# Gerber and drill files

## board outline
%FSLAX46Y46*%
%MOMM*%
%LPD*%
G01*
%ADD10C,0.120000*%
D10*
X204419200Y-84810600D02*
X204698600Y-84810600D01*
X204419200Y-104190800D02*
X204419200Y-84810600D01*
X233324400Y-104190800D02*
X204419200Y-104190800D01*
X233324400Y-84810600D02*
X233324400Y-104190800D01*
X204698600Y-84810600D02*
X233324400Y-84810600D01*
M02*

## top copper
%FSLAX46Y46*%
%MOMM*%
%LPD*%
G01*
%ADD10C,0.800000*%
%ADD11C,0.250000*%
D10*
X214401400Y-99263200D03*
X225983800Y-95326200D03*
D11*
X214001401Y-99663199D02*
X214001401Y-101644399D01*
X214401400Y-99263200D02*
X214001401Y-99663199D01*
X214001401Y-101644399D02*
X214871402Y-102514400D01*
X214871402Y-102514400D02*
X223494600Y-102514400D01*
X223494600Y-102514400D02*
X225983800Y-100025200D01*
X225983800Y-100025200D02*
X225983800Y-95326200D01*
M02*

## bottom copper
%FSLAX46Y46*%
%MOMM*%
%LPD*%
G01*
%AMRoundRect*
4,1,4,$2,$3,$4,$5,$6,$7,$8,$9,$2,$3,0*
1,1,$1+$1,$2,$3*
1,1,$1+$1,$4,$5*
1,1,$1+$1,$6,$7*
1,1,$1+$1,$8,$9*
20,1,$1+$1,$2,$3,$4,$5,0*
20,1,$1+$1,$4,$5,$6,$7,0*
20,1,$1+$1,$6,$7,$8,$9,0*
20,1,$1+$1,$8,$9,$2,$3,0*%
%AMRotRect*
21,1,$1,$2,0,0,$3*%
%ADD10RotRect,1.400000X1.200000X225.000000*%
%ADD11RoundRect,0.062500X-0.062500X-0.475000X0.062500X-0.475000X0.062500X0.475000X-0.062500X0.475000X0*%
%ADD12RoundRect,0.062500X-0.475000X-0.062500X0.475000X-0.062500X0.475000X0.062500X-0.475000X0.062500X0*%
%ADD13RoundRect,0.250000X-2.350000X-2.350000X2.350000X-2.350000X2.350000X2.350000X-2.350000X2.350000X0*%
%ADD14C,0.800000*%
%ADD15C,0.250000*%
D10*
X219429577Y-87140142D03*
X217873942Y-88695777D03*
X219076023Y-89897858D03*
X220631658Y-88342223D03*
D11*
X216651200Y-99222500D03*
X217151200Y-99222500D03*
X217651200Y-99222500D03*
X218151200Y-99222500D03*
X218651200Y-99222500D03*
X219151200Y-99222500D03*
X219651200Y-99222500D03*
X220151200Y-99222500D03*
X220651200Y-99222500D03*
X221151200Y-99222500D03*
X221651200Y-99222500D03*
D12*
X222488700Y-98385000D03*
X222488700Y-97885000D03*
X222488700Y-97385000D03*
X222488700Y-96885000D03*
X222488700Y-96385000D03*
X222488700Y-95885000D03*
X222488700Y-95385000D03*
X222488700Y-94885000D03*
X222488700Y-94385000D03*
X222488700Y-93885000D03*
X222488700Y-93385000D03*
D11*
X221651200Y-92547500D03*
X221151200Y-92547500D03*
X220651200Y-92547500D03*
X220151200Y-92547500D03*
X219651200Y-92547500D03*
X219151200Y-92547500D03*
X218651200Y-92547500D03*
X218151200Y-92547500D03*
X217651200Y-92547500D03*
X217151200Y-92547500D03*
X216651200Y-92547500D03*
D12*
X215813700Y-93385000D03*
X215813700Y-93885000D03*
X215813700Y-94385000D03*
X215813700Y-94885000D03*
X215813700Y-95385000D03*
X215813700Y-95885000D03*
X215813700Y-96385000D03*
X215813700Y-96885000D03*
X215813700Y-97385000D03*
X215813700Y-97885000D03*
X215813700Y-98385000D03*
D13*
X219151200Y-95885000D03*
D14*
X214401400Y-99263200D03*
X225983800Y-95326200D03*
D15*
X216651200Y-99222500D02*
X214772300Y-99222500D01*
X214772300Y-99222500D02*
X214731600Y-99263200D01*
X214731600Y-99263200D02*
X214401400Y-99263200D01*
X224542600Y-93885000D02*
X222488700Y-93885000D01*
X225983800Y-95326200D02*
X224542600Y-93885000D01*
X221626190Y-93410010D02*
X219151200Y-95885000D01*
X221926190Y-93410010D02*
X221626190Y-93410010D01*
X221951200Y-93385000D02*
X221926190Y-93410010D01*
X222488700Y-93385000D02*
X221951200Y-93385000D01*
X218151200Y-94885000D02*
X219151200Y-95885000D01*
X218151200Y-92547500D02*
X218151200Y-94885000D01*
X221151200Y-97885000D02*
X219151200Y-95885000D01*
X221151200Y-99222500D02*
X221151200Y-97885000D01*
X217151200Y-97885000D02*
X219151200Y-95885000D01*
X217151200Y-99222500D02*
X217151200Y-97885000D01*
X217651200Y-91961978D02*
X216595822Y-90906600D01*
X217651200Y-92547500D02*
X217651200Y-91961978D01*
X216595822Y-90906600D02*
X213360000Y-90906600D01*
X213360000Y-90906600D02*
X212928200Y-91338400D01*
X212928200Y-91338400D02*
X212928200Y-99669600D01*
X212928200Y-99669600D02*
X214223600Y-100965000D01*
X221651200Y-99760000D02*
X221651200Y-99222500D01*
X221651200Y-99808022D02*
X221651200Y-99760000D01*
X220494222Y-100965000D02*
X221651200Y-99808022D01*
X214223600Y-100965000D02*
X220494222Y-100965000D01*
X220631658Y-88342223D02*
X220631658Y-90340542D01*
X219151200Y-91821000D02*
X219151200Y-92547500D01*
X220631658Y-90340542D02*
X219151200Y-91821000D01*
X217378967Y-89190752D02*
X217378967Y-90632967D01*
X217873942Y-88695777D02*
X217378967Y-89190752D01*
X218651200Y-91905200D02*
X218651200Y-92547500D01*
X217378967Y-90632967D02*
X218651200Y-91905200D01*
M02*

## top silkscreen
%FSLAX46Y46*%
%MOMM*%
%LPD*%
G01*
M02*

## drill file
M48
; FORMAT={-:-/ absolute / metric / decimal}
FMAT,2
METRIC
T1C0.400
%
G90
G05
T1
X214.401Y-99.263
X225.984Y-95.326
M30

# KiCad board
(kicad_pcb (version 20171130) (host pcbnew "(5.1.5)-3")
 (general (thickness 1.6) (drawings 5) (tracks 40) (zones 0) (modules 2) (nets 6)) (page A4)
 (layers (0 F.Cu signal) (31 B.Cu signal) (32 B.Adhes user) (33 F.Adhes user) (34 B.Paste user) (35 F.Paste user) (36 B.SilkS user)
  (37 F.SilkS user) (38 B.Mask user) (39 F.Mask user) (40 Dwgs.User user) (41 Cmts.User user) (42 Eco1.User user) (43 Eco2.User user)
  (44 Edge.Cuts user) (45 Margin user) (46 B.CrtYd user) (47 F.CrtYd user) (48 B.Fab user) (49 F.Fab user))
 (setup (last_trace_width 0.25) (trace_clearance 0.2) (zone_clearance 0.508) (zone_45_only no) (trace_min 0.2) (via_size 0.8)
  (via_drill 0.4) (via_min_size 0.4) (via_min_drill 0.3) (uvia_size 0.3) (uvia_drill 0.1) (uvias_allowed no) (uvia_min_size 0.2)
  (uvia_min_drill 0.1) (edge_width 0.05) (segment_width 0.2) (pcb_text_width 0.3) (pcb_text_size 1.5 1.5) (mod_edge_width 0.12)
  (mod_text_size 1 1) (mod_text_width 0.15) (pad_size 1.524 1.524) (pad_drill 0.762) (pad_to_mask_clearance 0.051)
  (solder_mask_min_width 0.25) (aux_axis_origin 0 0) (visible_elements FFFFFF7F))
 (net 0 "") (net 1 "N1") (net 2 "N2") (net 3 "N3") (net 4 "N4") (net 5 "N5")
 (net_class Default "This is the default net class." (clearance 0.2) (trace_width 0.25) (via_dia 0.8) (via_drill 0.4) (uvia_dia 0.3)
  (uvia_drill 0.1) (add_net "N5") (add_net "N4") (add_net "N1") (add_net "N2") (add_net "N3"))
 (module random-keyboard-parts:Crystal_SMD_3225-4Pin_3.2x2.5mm (layer B.Cu) (at 219.2528 88.519 225)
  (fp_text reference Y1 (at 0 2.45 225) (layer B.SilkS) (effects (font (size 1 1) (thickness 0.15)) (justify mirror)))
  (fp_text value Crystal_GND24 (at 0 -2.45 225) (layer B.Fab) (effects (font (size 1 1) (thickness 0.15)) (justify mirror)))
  (pad 4 smd rect (at -1.1 0.85 225) (size 1.4 1.2) (layers B.Cu B.Paste B.Mask))
  (pad 3 smd rect (at 1.1 0.85 225) (size 1.4 1.2) (layers B.Cu B.Paste B.Mask) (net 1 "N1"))
  (pad 2 smd rect (at 1.1 -0.85 225) (size 1.4 1.2) (layers B.Cu B.Paste B.Mask))
  (pad 1 smd rect (at -1.1 -0.85 225) (size 1.4 1.2) (layers B.Cu B.Paste B.Mask) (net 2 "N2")))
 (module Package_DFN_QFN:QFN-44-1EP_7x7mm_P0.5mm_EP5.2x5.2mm (layer B.Cu) (at 219.1512 95.885)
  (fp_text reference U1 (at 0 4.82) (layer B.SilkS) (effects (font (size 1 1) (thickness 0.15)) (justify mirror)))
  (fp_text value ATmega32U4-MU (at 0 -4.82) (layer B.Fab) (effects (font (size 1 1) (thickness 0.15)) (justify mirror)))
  (pad 44 smd roundrect (at -2.5 3.3375) (size 0.25 1.075) (layers B.Cu B.Paste B.Mask) (roundrect_rratio 0.25) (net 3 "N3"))
  (pad 43 smd roundrect (at -2 3.3375) (size 0.25 1.075) (layers B.Cu B.Paste B.Mask) (roundrect_rratio 0.25) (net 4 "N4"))
  (pad 42 smd roundrect (at -1.5 3.3375) (size 0.25 1.075) (layers B.Cu B.Paste B.Mask) (roundrect_rratio 0.25))
  (pad 41 smd roundrect (at -1 3.3375) (size 0.25 1.075) (layers B.Cu B.Paste B.Mask) (roundrect_rratio 0.25))
  (pad 40 smd roundrect (at -0.5 3.3375) (size 0.25 1.075) (layers B.Cu B.Paste B.Mask) (roundrect_rratio 0.25))
  (pad 39 smd roundrect (at 0 3.3375) (size 0.25 1.075) (layers B.Cu B.Paste B.Mask) (roundrect_rratio 0.25))
  (pad 38 smd roundrect (at 0.5 3.3375) (size 0.25 1.075) (layers B.Cu B.Paste B.Mask) (roundrect_rratio 0.25))
  (pad 37 smd roundrect (at 1 3.3375) (size 0.25 1.075) (layers B.Cu B.Paste B.Mask) (roundrect_rratio 0.25))
  (pad 36 smd roundrect (at 1.5 3.3375) (size 0.25 1.075) (layers B.Cu B.Paste B.Mask) (roundrect_rratio 0.25))
  (pad 35 smd roundrect (at 2 3.3375) (size 0.25 1.075) (layers B.Cu B.Paste B.Mask) (roundrect_rratio 0.25) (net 4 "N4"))
  (pad 34 smd roundrect (at 2.5 3.3375) (size 0.25 1.075) (layers B.Cu B.Paste B.Mask) (roundrect_rratio 0.25) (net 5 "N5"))
  (pad 33 smd roundrect (at 3.3375 2.5) (size 1.075 0.25) (layers B.Cu B.Paste B.Mask) (roundrect_rratio 0.25))
  (pad 32 smd roundrect (at 3.3375 2) (size 1.075 0.25) (layers B.Cu B.Paste B.Mask) (roundrect_rratio 0.25))
  (pad 31 smd roundrect (at 3.3375 1.5) (size 1.075 0.25) (layers B.Cu B.Paste B.Mask) (roundrect_rratio 0.25))
  (pad 30 smd roundrect (at 3.3375 1) (size 1.075 0.25) (layers B.Cu B.Paste B.Mask) (roundrect_rratio 0.25))
  (pad 29 smd roundrect (at 3.3375 0.5) (size 1.075 0.25) (layers B.Cu B.Paste B.Mask) (roundrect_rratio 0.25))
  (pad 28 smd roundrect (at 3.3375 0) (size 1.075 0.25) (layers B.Cu B.Paste B.Mask) (roundrect_rratio 0.25))
  (pad 27 smd roundrect (at 3.3375 -0.5) (size 1.075 0.25) (layers B.Cu B.Paste B.Mask) (roundrect_rratio 0.25))
  (pad 26 smd roundrect (at 3.3375 -1) (size 1.075 0.25) (layers B.Cu B.Paste B.Mask) (roundrect_rratio 0.25))
  (pad 25 smd roundrect (at 3.3375 -1.5) (size 1.075 0.25) (layers B.Cu B.Paste B.Mask) (roundrect_rratio 0.25))
  (pad 24 smd roundrect (at 3.3375 -2) (size 1.075 0.25) (layers B.Cu B.Paste B.Mask) (roundrect_rratio 0.25) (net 3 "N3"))
  (pad 23 smd roundrect (at 3.3375 -2.5) (size 1.075 0.25) (layers B.Cu B.Paste B.Mask) (roundrect_rratio 0.25) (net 4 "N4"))
  (pad 22 smd roundrect (at 2.5 -3.3375) (size 0.25 1.075) (layers B.Cu B.Paste B.Mask) (roundrect_rratio 0.25))
  (pad 21 smd roundrect (at 2 -3.3375) (size 0.25 1.075) (layers B.Cu B.Paste B.Mask) (roundrect_rratio 0.25))
  (pad 20 smd roundrect (at 1.5 -3.3375) (size 0.25 1.075) (layers B.Cu B.Paste B.Mask) (roundrect_rratio 0.25))
  (pad 19 smd roundrect (at 1 -3.3375) (size 0.25 1.075) (layers B.Cu B.Paste B.Mask) (roundrect_rratio 0.25))
  (pad 18 smd roundrect (at 0.5 -3.3375) (size 0.25 1.075) (layers B.Cu B.Paste B.Mask) (roundrect_rratio 0.25))
  (pad 17 smd roundrect (at 0 -3.3375) (size 0.25 1.075) (layers B.Cu B.Paste B.Mask) (roundrect_rratio 0.25) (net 2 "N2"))
  (pad 16 smd roundrect (at -0.5 -3.3375) (size 0.25 1.075) (layers B.Cu B.Paste B.Mask) (roundrect_rratio 0.25) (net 1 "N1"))
  (pad 15 smd roundrect (at -1 -3.3375) (size 0.25 1.075) (layers B.Cu B.Paste B.Mask) (roundrect_rratio 0.25) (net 4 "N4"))
  (pad 14 smd roundrect (at -1.5 -3.3375) (size 0.25 1.075) (layers B.Cu B.Paste B.Mask) (roundrect_rratio 0.25) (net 5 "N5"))
  (pad 13 smd roundrect (at -2 -3.3375) (size 0.25 1.075) (layers B.Cu B.Paste B.Mask) (roundrect_rratio 0.25))
  (pad 12 smd roundrect (at -2.5 -3.3375) (size 0.25 1.075) (layers B.Cu B.Paste B.Mask) (roundrect_rratio 0.25))
  (pad 11 smd roundrect (at -3.3375 -2.5) (size 1.075 0.25) (layers B.Cu B.Paste B.Mask) (roundrect_rratio 0.25))
  (pad 10 smd roundrect (at -3.3375 -2) (size 1.075 0.25) (layers B.Cu B.Paste B.Mask) (roundrect_rratio 0.25))
  (pad 9 smd roundrect (at -3.3375 -1.5) (size 1.075 0.25) (layers B.Cu B.Paste B.Mask) (roundrect_rratio 0.25))
  (pad 8 smd roundrect (at -3.3375 -1) (size 1.075 0.25) (layers B.Cu B.Paste B.Mask) (roundrect_rratio 0.25))
  (pad 7 smd roundrect (at -3.3375 -0.5) (size 1.075 0.25) (layers B.Cu B.Paste B.Mask) (roundrect_rratio 0.25))
  (pad 6 smd roundrect (at -3.3375 0) (size 1.075 0.25) (layers B.Cu B.Paste B.Mask) (roundrect_rratio 0.25))
  (pad 5 smd roundrect (at -3.3375 0.5) (size 1.075 0.25) (layers B.Cu B.Paste B.Mask) (roundrect_rratio 0.25))
  (pad 4 smd roundrect (at -3.3375 1) (size 1.075 0.25) (layers B.Cu B.Paste B.Mask) (roundrect_rratio 0.25))
  (pad 3 smd roundrect (at -3.3375 1.5) (size 1.075 0.25) (layers B.Cu B.Paste B.Mask) (roundrect_rratio 0.25))
  (pad 2 smd roundrect (at -3.3375 2) (size 1.075 0.25) (layers B.Cu B.Paste B.Mask) (roundrect_rratio 0.25))
  (pad 1 smd roundrect (at -3.3375 2.5) (size 1.075 0.25) (layers B.Cu B.Paste B.Mask) (roundrect_rratio 0.25))
  (pad "" smd roundrect (at 1.95 -1.95) (size 1.05 1.05) (layers B.Paste) (roundrect_rratio 0.238095))
  (pad "" smd roundrect (at 1.95 -0.65) (size 1.05 1.05) (layers B.Paste) (roundrect_rratio 0.238095))
  (pad "" smd roundrect (at 1.95 0.65) (size 1.05 1.05) (layers B.Paste) (roundrect_rratio 0.238095))
  (pad "" smd roundrect (at 1.95 1.95) (size 1.05 1.05) (layers B.Paste) (roundrect_rratio 0.238095))
  (pad "" smd roundrect (at 0.65 -1.95) (size 1.05 1.05) (layers B.Paste) (roundrect_rratio 0.238095))
  (pad "" smd roundrect (at 0.65 -0.65) (size 1.05 1.05) (layers B.Paste) (roundrect_rratio 0.238095))
  (pad "" smd roundrect (at 0.65 0.65) (size 1.05 1.05) (layers B.Paste) (roundrect_rratio 0.238095))
  (pad "" smd roundrect (at 0.65 1.95) (size 1.05 1.05) (layers B.Paste) (roundrect_rratio 0.238095))
  (pad "" smd roundrect (at -0.65 -1.95) (size 1.05 1.05) (layers B.Paste) (roundrect_rratio 0.238095))
  (pad "" smd roundrect (at -0.65 -0.65) (size 1.05 1.05) (layers B.Paste) (roundrect_rratio 0.238095))
  (pad "" smd roundrect (at -0.65 0.65) (size 1.05 1.05) (layers B.Paste) (roundrect_rratio 0.238095))
  (pad "" smd roundrect (at -0.65 1.95) (size 1.05 1.05) (layers B.Paste) (roundrect_rratio 0.238095))
  (pad "" smd roundrect (at -1.95 -1.95) (size 1.05 1.05) (layers B.Paste) (roundrect_rratio 0.238095))
  (pad "" smd roundrect (at -1.95 -0.65) (size 1.05 1.05) (layers B.Paste) (roundrect_rratio 0.238095))
  (pad "" smd roundrect (at -1.95 0.65) (size 1.05 1.05) (layers B.Paste) (roundrect_rratio 0.238095))
  (pad "" smd roundrect (at -1.95 1.95) (size 1.05 1.05) (layers B.Paste) (roundrect_rratio 0.238095))
  (pad 45 smd roundrect (at 0 0) (size 5.2 5.2) (layers B.Cu B.Mask) (roundrect_rratio 0.048077) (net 4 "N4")))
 (gr_line (start 204.4192 84.8106) (end 204.6986 84.8106) (layer Edge.Cuts) (width 0.12))
 (gr_line (start 204.4192 104.1908) (end 204.4192 84.8106) (layer Edge.Cuts) (width 0.12))
 (gr_line (start 233.3244 104.1908) (end 204.4192 104.1908) (layer Edge.Cuts) (width 0.12))
 (gr_line (start 233.3244 84.8106) (end 233.3244 104.1908) (layer Edge.Cuts) (width 0.12))
 (gr_line (start 204.6986 84.8106) (end 233.3244 84.8106) (layer Edge.Cuts) (width 0.12))
 (segment (start 216.6512 99.2225) (end 214.7723 99.2225) (width 0.25) (layer B.Cu) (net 3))
 (via (at 214.4014 99.2632) (size 0.8) (drill 0.4) (layers F.Cu B.Cu) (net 3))
 (segment (start 214.7723 99.2225) (end 214.7316 99.2632) (width 0.25) (layer B.Cu) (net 3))
 (segment (start 214.7316 99.2632) (end 214.4014 99.2632) (width 0.25) (layer B.Cu) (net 3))
 (segment (start 214.001401 99.663199) (end 214.001401 101.644399) (width 0.25) (layer F.Cu) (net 3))
 (segment (start 214.4014 99.2632) (end 214.001401 99.663199) (width 0.25) (layer F.Cu) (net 3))
 (segment (start 214.001401 101.644399) (end 214.871402 102.5144) (width 0.25) (layer F.Cu) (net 3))
 (segment (start 214.871402 102.5144) (end 223.4946 102.5144) (width 0.25) (layer F.Cu) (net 3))
 (via (at 225.9838 95.3262) (size 0.8) (drill 0.4) (layers F.Cu B.Cu) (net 3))
 (segment (start 223.4946 102.5144) (end 225.9838 100.0252) (width 0.25) (layer F.Cu) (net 3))
 (segment (start 225.9838 100.0252) (end 225.9838 95.3262) (width 0.25) (layer F.Cu) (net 3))
 (segment (start 224.5426 93.885) (end 222.4887 93.885) (width 0.25) (layer B.Cu) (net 3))
 (segment (start 225.9838 95.3262) (end 224.5426 93.885) (width 0.25) (layer B.Cu) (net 3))
 (segment (start 221.62619 93.41001) (end 219.1512 95.885) (width 0.25) (layer B.Cu) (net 4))
 (segment (start 221.92619 93.41001) (end 221.62619 93.41001) (width 0.25) (layer B.Cu) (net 4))
 (segment (start 221.9512 93.385) (end 221.92619 93.41001) (width 0.25) (layer B.Cu) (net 4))
 (segment (start 222.4887 93.385) (end 221.9512 93.385) (width 0.25) (layer B.Cu) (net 4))
 (segment (start 218.1512 94.885) (end 219.1512 95.885) (width 0.25) (layer B.Cu) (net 4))
 (segment (start 218.1512 92.5475) (end 218.1512 94.885) (width 0.25) (layer B.Cu) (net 4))
 (segment (start 221.1512 97.885) (end 219.1512 95.885) (width 0.25) (layer B.Cu) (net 4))
 (segment (start 221.1512 99.2225) (end 221.1512 97.885) (width 0.25) (layer B.Cu) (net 4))
 (segment (start 217.1512 97.885) (end 219.1512 95.885) (width 0.25) (layer B.Cu) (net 4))
 (segment (start 217.1512 99.2225) (end 217.1512 97.885) (width 0.25) (layer B.Cu) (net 4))
 (segment (start 217.6512 91.961978) (end 216.595822 90.9066) (width 0.25) (layer B.Cu) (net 5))
 (segment (start 217.6512 92.5475) (end 217.6512 91.961978) (width 0.25) (layer B.Cu) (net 5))
 (segment (start 216.595822 90.9066) (end 213.36 90.9066) (width 0.25) (layer B.Cu) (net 5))
 (segment (start 213.36 90.9066) (end 212.9282 91.3384) (width 0.25) (layer B.Cu) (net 5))
 (segment (start 212.9282 91.3384) (end 212.9282 99.6696) (width 0.25) (layer B.Cu) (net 5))
 (segment (start 212.9282 99.6696) (end 214.2236 100.965) (width 0.25) (layer B.Cu) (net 5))
 (segment (start 221.6512 99.76) (end 221.6512 99.2225) (width 0.25) (layer B.Cu) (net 5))
 (segment (start 221.6512 99.808022) (end 221.6512 99.76) (width 0.25) (layer B.Cu) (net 5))
 (segment (start 220.494222 100.965) (end 221.6512 99.808022) (width 0.25) (layer B.Cu) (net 5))
 (segment (start 214.2236 100.965) (end 220.494222 100.965) (width 0.25) (layer B.Cu) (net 5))
 (segment (start 220.631658 88.342223) (end 220.631658 90.340542) (width 0.25) (layer B.Cu) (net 2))
 (segment (start 219.1512 91.821) (end 219.1512 92.5475) (width 0.25) (layer B.Cu) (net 2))
 (segment (start 220.631658 90.340542) (end 219.1512 91.821) (width 0.25) (layer B.Cu) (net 2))
 (segment (start 217.378967 89.190752) (end 217.378967 90.632967) (width 0.25) (layer B.Cu) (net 1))
 (segment (start 217.873942 88.695777) (end 217.378967 89.190752) (width 0.25) (layer B.Cu) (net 1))
 (segment (start 218.6512 91.9052) (end 218.6512 92.5475) (width 0.25) (layer B.Cu) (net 1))
 (segment (start 217.378967 90.632967) (end 218.6512 91.9052) (width 0.25) (layer B.Cu) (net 1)))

